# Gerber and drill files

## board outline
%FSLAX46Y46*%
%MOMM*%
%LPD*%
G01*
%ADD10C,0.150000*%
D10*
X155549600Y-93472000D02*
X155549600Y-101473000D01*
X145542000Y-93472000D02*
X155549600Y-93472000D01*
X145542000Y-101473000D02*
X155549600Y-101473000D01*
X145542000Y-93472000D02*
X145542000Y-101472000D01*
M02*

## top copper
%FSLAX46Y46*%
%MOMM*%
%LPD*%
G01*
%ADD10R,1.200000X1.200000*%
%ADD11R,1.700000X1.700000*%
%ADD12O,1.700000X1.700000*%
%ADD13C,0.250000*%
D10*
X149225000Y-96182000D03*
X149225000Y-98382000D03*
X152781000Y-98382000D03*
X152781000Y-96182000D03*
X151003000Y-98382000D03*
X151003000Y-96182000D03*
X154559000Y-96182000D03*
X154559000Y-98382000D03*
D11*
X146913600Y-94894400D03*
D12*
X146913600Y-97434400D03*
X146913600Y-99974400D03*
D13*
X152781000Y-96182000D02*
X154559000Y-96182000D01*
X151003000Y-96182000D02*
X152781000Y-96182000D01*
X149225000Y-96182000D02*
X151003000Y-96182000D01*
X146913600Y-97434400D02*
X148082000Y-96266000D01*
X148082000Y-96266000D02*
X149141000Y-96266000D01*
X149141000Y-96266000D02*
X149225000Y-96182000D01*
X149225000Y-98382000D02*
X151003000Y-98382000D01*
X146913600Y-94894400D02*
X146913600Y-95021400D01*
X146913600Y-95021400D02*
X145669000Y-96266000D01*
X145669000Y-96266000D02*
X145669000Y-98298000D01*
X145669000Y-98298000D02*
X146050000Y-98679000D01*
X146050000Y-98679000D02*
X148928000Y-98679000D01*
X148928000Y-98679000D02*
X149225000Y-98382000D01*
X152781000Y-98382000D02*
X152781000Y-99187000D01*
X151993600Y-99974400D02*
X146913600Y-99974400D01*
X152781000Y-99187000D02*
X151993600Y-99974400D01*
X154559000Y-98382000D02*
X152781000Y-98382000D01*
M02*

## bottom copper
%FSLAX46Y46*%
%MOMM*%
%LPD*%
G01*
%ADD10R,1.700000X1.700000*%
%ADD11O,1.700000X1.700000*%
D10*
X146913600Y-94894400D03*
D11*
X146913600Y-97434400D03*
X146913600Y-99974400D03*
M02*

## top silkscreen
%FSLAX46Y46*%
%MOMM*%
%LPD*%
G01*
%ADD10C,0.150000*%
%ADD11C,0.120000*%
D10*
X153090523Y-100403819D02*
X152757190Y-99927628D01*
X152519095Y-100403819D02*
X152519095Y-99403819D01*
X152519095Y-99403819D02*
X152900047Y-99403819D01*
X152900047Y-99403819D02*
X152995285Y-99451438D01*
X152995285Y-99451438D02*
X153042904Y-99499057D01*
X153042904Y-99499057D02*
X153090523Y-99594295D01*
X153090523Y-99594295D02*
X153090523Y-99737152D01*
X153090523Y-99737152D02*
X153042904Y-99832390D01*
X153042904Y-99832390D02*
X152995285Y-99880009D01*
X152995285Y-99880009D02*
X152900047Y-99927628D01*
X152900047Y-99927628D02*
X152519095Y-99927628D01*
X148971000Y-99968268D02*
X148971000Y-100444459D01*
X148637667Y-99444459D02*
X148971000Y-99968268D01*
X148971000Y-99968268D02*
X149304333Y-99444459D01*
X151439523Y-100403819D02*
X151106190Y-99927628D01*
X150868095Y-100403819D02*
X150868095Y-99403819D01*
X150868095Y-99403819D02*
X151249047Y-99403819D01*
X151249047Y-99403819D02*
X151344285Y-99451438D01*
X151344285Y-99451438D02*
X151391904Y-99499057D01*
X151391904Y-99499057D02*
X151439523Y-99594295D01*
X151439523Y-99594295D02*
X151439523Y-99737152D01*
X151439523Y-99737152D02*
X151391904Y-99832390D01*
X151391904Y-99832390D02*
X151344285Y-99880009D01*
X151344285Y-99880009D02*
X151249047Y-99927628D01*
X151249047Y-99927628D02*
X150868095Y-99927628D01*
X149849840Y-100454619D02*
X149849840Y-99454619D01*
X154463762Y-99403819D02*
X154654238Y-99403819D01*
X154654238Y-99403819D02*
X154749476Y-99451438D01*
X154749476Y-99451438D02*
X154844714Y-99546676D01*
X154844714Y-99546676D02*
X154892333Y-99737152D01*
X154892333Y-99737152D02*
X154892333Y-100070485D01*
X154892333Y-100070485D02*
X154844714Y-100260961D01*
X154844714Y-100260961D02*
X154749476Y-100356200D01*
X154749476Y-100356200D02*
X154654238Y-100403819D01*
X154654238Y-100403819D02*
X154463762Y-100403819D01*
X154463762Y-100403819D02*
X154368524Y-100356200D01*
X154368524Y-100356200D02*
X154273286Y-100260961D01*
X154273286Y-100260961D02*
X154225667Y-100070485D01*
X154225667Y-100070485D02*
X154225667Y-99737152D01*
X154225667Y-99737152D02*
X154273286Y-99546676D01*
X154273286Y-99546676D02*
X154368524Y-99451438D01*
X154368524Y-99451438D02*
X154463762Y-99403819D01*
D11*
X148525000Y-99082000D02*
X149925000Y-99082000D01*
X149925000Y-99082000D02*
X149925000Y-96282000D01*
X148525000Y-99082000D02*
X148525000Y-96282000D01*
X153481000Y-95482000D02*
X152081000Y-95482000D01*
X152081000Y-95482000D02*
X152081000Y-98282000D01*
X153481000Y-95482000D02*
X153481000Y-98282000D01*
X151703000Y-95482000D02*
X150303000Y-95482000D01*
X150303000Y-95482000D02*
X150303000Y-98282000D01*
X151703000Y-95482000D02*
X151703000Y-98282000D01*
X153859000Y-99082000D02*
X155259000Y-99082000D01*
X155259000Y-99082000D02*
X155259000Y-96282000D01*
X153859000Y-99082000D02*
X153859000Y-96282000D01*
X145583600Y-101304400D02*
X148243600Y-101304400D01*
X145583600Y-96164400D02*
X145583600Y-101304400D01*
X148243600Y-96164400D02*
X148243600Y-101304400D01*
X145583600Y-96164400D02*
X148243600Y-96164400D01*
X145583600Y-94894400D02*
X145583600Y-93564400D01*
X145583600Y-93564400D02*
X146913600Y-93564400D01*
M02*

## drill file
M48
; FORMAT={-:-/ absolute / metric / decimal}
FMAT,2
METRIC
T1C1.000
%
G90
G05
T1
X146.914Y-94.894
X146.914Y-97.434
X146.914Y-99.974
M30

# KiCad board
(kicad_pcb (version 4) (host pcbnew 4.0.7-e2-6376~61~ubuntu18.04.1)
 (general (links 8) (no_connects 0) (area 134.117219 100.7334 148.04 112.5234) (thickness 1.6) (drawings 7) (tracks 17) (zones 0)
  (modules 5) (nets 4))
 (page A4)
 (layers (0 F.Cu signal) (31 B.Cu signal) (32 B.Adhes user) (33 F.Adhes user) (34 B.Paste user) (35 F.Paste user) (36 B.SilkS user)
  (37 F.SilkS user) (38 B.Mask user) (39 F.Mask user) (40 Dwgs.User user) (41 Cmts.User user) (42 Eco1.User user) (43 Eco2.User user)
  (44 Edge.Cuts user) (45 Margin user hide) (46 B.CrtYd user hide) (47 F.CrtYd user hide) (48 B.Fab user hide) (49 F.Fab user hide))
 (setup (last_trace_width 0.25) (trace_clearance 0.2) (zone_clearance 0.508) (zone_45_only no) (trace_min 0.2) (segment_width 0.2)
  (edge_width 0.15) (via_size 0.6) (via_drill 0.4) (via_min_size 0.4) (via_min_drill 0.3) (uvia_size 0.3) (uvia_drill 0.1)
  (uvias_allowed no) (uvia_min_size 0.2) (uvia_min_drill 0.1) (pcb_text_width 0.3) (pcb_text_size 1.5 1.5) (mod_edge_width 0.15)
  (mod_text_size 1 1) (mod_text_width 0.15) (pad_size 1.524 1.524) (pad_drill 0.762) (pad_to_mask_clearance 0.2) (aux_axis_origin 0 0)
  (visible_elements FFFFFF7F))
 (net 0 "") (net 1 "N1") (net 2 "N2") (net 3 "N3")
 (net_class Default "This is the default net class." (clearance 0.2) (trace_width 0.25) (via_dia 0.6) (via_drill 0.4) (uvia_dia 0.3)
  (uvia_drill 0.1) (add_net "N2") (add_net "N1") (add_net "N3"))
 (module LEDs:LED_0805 (layer F.Cu) (at 149.225 97.282 90)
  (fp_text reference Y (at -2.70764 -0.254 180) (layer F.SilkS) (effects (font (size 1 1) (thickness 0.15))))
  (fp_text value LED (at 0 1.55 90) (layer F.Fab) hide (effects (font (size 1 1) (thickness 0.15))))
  (fp_line (start -1.8 -0.7) (end -1.8 0.7) (layer F.SilkS) (width 0.12))
  (fp_line (start -1.8 0.7) (end 1 0.7) (layer F.SilkS) (width 0.12))
  (fp_line (start -1.8 -0.7) (end 1 -0.7) (layer F.SilkS) (width 0.12))
  (pad 2 smd rect (at 1.1 0 270) (size 1.2 1.2) (layers F.Cu F.Paste F.Mask) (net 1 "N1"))
  (pad 1 smd rect (at -1.1 0 270) (size 1.2 1.2) (layers F.Cu F.Paste F.Mask) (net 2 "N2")))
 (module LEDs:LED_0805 (layer F.Cu) (at 152.781 97.282 270)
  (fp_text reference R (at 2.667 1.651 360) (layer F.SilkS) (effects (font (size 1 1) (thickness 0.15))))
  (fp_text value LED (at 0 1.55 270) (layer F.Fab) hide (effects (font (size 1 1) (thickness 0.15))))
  (fp_line (start -1.8 -0.7) (end -1.8 0.7) (layer F.SilkS) (width 0.12))
  (fp_line (start -1.8 0.7) (end 1 0.7) (layer F.SilkS) (width 0.12))
  (fp_line (start -1.8 -0.7) (end 1 -0.7) (layer F.SilkS) (width 0.12))
  (pad 2 smd rect (at 1.1 0 90) (size 1.2 1.2) (layers F.Cu F.Paste F.Mask) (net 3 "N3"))
  (pad 1 smd rect (at -1.1 0 90) (size 1.2 1.2) (layers F.Cu F.Paste F.Mask) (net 1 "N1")))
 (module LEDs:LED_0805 (layer F.Cu) (at 151.003 97.282 270)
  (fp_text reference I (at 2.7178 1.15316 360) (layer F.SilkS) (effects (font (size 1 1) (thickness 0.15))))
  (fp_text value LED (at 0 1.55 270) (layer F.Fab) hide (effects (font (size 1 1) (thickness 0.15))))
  (fp_line (start -1.8 -0.7) (end -1.8 0.7) (layer F.SilkS) (width 0.12))
  (fp_line (start -1.8 0.7) (end 1 0.7) (layer F.SilkS) (width 0.12))
  (fp_line (start -1.8 -0.7) (end 1 -0.7) (layer F.SilkS) (width 0.12))
  (pad 2 smd rect (at 1.1 0 90) (size 1.2 1.2) (layers F.Cu F.Paste F.Mask) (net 2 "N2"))
  (pad 1 smd rect (at -1.1 0 90) (size 1.2 1.2) (layers F.Cu F.Paste F.Mask) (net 1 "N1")))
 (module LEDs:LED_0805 (layer F.Cu) (at 154.559 97.282 90)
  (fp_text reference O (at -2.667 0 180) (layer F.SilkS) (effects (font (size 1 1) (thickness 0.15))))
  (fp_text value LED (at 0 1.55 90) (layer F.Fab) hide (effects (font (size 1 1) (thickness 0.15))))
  (fp_line (start -1.8 -0.7) (end -1.8 0.7) (layer F.SilkS) (width 0.12))
  (fp_line (start -1.8 0.7) (end 1 0.7) (layer F.SilkS) (width 0.12))
  (fp_line (start -1.8 -0.7) (end 1 -0.7) (layer F.SilkS) (width 0.12))
  (pad 2 smd rect (at 1.1 0 270) (size 1.2 1.2) (layers F.Cu F.Paste F.Mask) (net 1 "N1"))
  (pad 1 smd rect (at -1.1 0 270) (size 1.2 1.2) (layers F.Cu F.Paste F.Mask) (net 3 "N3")))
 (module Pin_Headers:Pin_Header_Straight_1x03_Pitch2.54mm (layer F.Cu) (at 146.9136 94.8944)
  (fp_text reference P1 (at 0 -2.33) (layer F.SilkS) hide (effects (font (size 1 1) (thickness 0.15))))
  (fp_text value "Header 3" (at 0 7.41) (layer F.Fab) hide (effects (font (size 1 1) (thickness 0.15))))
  (fp_line (start -1.33 6.41) (end 1.33 6.41) (layer F.SilkS) (width 0.12))
  (fp_line (start -1.33 1.27) (end -1.33 6.41) (layer F.SilkS) (width 0.12))
  (fp_line (start 1.33 1.27) (end 1.33 6.41) (layer F.SilkS) (width 0.12))
  (fp_line (start -1.33 1.27) (end 1.33 1.27) (layer F.SilkS) (width 0.12))
  (fp_line (start -1.33 0) (end -1.33 -1.33) (layer F.SilkS) (width 0.12))
  (fp_line (start -1.33 -1.33) (end 0 -1.33) (layer F.SilkS) (width 0.12))
  (pad 1 thru_hole rect (at 0 0) (size 1.7 1.7) (drill 1) (layers *.Cu *.Mask) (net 2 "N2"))
  (pad 2 thru_hole oval (at 0 2.54) (size 1.7 1.7) (drill 1) (layers *.Cu *.Mask) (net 1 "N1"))
  (pad 3 thru_hole oval (at 0 5.08) (size 1.7 1.7) (drill 1) (layers *.Cu *.Mask) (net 3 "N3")))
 (gr_line (start 155.5496 93.472) (end 155.5496 101.473) (angle 90) (layer Edge.Cuts) (width 0.15))
 (gr_line (start 145.542 93.472) (end 155.5496 93.472) (angle 90) (layer Edge.Cuts) (width 0.15))
 (gr_line (start 145.542 101.473) (end 155.5496 101.473) (angle 90) (layer Edge.Cuts) (width 0.15))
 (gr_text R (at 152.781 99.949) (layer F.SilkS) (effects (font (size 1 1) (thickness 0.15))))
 (gr_line (start 145.542 93.472) (end 145.542 101.472) (angle 90) (layer Edge.Cuts) (width 0.15))
 (segment (start 152.781 96.182) (end 154.559 96.182) (width 0.25) (layer F.Cu) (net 1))
 (segment (start 151.003 96.182) (end 152.781 96.182) (width 0.25) (layer F.Cu) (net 1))
 (segment (start 149.225 96.182) (end 151.003 96.182) (width 0.25) (layer F.Cu) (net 1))
 (segment (start 146.9136 97.4344) (end 148.082 96.266) (width 0.25) (layer F.Cu) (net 1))
 (segment (start 148.082 96.266) (end 149.141 96.266) (width 0.25) (layer F.Cu) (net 1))
 (segment (start 149.141 96.266) (end 149.225 96.182) (width 0.25) (layer F.Cu) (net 1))
 (segment (start 149.225 98.382) (end 151.003 98.382) (width 0.25) (layer F.Cu) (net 2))
 (segment (start 146.9136 94.8944) (end 146.9136 95.0214) (width 0.25) (layer F.Cu) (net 2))
 (segment (start 146.9136 95.0214) (end 145.669 96.266) (width 0.25) (layer F.Cu) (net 2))
 (segment (start 145.669 96.266) (end 145.669 98.298) (width 0.25) (layer F.Cu) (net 2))
 (segment (start 145.669 98.298) (end 146.05 98.679) (width 0.25) (layer F.Cu) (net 2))
 (segment (start 146.05 98.679) (end 148.928 98.679) (width 0.25) (layer F.Cu) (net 2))
 (segment (start 148.928 98.679) (end 149.225 98.382) (width 0.25) (layer F.Cu) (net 2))
 (segment (start 152.781 98.382) (end 152.781 99.187) (width 0.25) (layer F.Cu) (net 3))
 (segment (start 151.9936 99.9744) (end 146.9136 99.9744) (width 0.25) (layer F.Cu) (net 3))
 (segment (start 152.781 99.187) (end 151.9936 99.9744) (width 0.25) (layer F.Cu) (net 3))
 (segment (start 154.559 98.382) (end 152.781 98.382) (width 0.25) (layer F.Cu) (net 3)))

